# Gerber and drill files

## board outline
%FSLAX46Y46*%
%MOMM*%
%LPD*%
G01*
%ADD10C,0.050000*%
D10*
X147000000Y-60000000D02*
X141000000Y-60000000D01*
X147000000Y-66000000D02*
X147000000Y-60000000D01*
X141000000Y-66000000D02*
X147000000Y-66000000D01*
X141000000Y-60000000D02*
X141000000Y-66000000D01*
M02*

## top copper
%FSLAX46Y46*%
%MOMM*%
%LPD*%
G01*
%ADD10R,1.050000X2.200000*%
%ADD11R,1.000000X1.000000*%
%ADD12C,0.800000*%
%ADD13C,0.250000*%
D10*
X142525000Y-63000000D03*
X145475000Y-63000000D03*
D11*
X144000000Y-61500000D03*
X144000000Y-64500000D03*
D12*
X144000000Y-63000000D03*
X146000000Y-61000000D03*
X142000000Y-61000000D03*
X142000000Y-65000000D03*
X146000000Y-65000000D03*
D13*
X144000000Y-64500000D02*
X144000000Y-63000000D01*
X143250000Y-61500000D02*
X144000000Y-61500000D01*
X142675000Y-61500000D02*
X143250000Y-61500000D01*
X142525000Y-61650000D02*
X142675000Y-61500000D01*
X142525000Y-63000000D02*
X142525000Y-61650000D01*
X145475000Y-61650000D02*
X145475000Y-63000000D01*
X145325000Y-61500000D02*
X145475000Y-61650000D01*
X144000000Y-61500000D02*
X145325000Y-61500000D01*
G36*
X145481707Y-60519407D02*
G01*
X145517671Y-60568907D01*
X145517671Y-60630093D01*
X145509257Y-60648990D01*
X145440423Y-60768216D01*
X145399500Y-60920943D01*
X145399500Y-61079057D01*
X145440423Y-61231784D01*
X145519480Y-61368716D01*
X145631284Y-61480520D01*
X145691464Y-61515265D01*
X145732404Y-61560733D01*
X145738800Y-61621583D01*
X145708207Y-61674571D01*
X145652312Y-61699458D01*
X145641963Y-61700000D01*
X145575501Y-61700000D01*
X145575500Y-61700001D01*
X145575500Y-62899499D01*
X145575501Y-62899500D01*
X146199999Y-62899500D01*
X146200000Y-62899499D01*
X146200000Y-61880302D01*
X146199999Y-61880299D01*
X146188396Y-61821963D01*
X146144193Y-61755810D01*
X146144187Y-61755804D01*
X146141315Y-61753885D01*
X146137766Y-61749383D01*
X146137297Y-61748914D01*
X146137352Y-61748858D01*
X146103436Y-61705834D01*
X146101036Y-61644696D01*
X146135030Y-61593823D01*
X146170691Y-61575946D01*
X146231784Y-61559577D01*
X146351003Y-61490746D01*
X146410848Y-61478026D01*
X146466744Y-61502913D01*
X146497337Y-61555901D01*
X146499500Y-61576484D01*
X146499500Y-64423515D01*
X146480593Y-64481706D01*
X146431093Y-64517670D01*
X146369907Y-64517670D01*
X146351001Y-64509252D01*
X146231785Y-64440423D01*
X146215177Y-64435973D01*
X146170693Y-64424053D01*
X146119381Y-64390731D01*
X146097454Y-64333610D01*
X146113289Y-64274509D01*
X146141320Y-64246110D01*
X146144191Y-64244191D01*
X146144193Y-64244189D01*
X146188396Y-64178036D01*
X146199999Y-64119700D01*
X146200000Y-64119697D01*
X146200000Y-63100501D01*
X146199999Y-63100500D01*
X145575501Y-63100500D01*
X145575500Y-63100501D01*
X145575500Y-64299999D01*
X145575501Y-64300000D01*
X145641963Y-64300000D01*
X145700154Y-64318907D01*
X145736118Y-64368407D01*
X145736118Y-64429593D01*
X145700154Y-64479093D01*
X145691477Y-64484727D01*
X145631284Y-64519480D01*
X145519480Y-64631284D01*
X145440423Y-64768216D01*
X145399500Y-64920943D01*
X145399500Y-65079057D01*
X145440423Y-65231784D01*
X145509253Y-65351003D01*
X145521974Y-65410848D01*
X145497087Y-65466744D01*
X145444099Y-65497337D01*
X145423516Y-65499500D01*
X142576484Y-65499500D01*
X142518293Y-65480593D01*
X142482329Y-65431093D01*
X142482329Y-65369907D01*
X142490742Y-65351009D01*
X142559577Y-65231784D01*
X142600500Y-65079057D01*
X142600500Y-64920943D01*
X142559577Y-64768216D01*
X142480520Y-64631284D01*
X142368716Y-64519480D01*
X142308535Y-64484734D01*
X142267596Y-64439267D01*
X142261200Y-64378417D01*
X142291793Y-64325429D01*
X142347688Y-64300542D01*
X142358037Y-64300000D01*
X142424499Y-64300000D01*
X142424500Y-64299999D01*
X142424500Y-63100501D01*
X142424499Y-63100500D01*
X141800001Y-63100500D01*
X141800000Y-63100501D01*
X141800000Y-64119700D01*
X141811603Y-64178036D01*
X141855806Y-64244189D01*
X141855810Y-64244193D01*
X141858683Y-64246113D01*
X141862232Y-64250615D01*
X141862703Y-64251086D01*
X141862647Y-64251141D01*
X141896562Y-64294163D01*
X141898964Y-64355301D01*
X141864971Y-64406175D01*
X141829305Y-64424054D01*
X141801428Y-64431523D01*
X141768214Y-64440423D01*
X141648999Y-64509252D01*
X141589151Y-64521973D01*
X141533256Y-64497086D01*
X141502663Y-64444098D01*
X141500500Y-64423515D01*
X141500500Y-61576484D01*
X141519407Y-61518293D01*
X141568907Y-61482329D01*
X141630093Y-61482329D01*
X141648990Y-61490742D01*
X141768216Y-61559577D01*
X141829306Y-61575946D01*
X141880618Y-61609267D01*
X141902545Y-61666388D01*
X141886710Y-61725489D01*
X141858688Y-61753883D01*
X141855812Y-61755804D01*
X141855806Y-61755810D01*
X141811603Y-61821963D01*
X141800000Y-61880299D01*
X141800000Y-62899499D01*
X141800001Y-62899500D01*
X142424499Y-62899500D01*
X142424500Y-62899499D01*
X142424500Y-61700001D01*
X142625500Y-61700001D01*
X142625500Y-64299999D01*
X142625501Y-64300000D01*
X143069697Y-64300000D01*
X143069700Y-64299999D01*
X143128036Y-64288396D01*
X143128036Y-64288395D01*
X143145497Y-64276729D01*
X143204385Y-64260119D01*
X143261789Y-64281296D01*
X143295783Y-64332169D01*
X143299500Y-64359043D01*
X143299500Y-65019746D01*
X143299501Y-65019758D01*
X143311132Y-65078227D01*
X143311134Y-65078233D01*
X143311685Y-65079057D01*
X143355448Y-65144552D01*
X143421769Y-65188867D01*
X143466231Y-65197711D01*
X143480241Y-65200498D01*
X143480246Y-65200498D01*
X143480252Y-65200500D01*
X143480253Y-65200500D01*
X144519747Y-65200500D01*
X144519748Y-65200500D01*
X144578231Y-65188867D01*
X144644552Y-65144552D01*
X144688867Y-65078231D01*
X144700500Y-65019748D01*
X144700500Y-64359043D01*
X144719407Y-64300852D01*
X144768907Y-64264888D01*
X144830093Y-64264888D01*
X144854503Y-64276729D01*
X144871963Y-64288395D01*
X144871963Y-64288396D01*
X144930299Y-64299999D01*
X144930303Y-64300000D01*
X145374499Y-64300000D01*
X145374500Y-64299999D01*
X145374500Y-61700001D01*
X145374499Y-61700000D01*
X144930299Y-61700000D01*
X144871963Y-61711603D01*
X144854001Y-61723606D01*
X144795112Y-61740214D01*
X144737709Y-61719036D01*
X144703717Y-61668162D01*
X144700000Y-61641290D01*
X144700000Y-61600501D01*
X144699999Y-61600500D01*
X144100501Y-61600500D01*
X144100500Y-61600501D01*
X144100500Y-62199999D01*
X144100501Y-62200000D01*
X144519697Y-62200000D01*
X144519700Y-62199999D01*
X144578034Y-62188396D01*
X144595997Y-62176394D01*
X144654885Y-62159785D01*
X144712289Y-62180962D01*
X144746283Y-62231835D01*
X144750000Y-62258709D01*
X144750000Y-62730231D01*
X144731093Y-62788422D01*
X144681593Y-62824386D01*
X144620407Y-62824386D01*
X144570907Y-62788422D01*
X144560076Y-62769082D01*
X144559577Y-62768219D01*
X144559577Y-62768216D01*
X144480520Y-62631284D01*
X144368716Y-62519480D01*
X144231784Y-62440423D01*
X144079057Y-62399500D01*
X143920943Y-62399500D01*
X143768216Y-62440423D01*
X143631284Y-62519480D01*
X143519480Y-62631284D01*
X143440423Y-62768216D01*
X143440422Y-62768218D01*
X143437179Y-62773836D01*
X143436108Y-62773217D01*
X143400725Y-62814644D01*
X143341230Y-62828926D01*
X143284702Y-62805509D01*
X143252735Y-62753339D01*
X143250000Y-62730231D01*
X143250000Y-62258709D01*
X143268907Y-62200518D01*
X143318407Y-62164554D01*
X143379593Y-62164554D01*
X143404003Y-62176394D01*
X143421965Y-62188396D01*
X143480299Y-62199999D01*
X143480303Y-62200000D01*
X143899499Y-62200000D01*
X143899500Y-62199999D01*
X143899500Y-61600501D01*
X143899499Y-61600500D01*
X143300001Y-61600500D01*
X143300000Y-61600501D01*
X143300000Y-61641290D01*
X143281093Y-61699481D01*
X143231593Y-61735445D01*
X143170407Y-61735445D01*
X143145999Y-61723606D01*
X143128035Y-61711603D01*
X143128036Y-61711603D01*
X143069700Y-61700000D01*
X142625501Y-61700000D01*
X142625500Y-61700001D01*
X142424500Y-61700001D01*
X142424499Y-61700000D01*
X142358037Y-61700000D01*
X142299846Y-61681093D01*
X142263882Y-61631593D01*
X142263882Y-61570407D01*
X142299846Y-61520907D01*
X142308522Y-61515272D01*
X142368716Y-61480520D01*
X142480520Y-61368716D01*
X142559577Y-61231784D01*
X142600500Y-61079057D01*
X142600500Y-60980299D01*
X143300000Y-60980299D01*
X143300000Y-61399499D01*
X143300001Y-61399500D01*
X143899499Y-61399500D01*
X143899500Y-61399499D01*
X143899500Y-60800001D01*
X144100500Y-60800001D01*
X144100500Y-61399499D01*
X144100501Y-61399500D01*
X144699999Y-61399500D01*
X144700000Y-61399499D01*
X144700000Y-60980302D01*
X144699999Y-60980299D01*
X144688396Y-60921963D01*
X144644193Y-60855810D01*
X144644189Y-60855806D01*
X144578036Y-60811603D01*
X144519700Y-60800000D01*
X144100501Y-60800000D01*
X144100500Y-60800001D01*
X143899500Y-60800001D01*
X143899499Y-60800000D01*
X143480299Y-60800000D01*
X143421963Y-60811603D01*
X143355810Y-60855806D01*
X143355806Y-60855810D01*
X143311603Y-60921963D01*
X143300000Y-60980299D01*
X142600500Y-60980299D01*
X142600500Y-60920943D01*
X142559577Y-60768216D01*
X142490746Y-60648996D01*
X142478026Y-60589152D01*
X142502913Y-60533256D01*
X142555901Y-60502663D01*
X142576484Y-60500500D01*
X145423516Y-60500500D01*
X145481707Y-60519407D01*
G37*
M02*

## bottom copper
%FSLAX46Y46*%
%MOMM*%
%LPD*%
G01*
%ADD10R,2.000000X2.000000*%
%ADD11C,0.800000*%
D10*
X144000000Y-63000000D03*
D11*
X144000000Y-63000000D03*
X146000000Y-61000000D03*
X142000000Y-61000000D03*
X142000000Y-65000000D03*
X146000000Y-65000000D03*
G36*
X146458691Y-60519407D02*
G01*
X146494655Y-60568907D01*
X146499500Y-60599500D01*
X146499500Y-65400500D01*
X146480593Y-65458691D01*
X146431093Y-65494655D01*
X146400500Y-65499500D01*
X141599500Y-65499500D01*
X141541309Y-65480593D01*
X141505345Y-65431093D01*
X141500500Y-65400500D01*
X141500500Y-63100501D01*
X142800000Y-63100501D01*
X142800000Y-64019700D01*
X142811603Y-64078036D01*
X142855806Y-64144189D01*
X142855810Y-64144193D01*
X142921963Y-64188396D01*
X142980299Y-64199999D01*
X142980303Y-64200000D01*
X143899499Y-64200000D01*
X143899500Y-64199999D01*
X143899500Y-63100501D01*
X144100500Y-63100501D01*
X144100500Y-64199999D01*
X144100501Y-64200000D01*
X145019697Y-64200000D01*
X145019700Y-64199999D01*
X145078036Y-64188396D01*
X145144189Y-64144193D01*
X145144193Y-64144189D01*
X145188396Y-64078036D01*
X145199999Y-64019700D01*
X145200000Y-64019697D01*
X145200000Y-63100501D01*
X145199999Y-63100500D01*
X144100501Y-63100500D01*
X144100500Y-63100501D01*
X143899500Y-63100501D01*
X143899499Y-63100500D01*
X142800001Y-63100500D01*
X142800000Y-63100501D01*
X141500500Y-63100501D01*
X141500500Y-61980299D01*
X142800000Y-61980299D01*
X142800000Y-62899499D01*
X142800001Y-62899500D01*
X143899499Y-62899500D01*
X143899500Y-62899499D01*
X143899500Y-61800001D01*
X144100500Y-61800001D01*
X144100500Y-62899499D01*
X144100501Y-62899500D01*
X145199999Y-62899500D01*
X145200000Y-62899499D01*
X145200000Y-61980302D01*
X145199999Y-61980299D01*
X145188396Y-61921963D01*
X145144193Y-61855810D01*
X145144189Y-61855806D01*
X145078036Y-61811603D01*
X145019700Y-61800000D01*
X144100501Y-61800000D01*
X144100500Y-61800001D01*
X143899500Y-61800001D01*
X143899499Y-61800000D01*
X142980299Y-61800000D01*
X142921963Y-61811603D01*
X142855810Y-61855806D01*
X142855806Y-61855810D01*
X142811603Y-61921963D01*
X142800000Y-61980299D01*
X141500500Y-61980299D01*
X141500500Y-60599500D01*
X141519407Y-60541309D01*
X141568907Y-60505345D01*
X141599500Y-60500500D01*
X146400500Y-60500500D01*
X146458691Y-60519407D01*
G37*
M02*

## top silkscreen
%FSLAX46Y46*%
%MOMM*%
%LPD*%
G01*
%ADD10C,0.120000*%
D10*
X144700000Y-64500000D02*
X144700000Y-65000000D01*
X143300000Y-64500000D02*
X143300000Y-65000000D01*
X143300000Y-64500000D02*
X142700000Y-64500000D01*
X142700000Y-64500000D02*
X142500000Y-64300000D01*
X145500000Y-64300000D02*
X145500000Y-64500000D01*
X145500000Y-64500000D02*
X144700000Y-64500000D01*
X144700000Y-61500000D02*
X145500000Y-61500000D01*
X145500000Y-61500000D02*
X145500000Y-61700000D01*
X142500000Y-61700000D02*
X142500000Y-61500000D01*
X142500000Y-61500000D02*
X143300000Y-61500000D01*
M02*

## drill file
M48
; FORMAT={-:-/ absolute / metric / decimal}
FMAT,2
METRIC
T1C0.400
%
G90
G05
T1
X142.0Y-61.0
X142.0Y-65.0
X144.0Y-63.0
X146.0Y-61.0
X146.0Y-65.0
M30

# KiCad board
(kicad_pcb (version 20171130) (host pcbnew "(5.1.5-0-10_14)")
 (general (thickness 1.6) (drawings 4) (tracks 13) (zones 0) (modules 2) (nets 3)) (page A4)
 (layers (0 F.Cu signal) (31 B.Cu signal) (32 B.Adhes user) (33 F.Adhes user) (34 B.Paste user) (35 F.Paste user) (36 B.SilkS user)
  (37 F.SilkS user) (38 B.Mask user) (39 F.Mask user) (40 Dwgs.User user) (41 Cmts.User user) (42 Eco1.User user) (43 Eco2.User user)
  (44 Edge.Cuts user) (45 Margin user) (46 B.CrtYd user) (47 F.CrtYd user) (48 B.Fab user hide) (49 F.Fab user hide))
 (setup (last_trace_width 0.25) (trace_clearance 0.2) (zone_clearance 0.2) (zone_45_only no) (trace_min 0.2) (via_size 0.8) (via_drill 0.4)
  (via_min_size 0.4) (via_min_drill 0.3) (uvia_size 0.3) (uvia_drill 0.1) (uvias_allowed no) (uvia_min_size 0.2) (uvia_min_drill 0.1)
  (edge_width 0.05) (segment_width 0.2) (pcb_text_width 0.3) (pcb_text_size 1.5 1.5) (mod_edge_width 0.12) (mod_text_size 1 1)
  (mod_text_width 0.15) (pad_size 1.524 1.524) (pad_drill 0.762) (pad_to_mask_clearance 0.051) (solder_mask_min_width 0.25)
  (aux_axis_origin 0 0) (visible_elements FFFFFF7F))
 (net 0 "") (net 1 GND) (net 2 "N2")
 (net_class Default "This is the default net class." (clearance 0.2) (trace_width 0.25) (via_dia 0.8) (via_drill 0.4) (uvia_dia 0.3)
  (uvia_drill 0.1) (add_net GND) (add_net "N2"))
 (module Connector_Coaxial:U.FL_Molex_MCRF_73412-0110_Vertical (layer F.Cu) (at 144 63)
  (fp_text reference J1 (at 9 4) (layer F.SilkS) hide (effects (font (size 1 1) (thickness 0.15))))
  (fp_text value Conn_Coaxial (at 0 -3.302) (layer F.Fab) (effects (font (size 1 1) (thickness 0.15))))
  (fp_line (start 0.7 1.5) (end 0.7 2) (layer F.SilkS) (width 0.12))
  (fp_line (start -0.7 1.5) (end -0.7 2) (layer F.SilkS) (width 0.12))
  (fp_line (start -0.7 1.5) (end -1.3 1.5) (layer F.SilkS) (width 0.12))
  (fp_line (start -1.3 1.5) (end -1.5 1.3) (layer F.SilkS) (width 0.12))
  (fp_line (start 1.5 1.3) (end 1.5 1.5) (layer F.SilkS) (width 0.12))
  (fp_line (start 1.5 1.5) (end 0.7 1.5) (layer F.SilkS) (width 0.12))
  (fp_line (start 0.7 -1.5) (end 1.5 -1.5) (layer F.SilkS) (width 0.12))
  (fp_line (start 1.5 -1.5) (end 1.5 -1.3) (layer F.SilkS) (width 0.12))
  (fp_line (start -1.5 -1.3) (end -1.5 -1.5) (layer F.SilkS) (width 0.12))
  (fp_line (start -1.5 -1.5) (end -0.7 -1.5) (layer F.SilkS) (width 0.12))
  (pad 2 smd rect (at -1.475 0) (size 1.05 2.2) (layers F.Cu F.Paste F.Mask) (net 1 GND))
  (pad 2 smd rect (at 1.475 0) (size 1.05 2.2) (layers F.Cu F.Paste F.Mask) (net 1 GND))
  (pad 2 smd rect (at 0 -1.5) (size 1 1) (layers F.Cu F.Paste F.Mask) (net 1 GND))
  (pad 1 smd rect (at 0 1.5) (size 1 1) (layers F.Cu F.Paste F.Mask) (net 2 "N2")))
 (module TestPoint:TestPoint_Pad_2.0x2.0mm (layer B.Cu) (at 144 63)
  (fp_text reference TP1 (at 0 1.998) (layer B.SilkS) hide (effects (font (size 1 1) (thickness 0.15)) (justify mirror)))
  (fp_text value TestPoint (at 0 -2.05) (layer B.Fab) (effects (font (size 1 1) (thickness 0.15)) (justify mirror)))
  (pad 1 smd rect (at 0 0) (size 2 2) (layers B.Cu B.Mask) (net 2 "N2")))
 (gr_line (start 147 60) (end 141 60) (layer Edge.Cuts) (width 0.05))
 (gr_line (start 147 66) (end 147 60) (layer Edge.Cuts) (width 0.05))
 (gr_line (start 141 66) (end 147 66) (layer Edge.Cuts) (width 0.05))
 (gr_line (start 141 60) (end 141 66) (layer Edge.Cuts) (width 0.05))
 (via (at 144 63) (size 0.8) (drill 0.4) (layers F.Cu B.Cu) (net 2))
 (segment (start 144 64.5) (end 144 63) (width 0.25) (layer F.Cu) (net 2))
 (via (at 146 61) (size 0.8) (drill 0.4) (layers F.Cu B.Cu) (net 2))
 (via (at 142 61) (size 0.8) (drill 0.4) (layers F.Cu B.Cu) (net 2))
 (via (at 142 65) (size 0.8) (drill 0.4) (layers F.Cu B.Cu) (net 2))
 (via (at 146 65) (size 0.8) (drill 0.4) (layers F.Cu B.Cu) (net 2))
 (segment (start 143.25 61.5) (end 144 61.5) (width 0.25) (layer F.Cu) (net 1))
 (segment (start 142.675 61.5) (end 143.25 61.5) (width 0.25) (layer F.Cu) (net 1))
 (segment (start 142.525 61.65) (end 142.675 61.5) (width 0.25) (layer F.Cu) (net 1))
 (segment (start 142.525 63) (end 142.525 61.65) (width 0.25) (layer F.Cu) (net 1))
 (segment (start 145.475 61.65) (end 145.475 63) (width 0.25) (layer F.Cu) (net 1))
 (segment (start 145.325 61.5) (end 145.475 61.65) (width 0.25) (layer F.Cu) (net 1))
 (segment (start 144 61.5) (end 145.325 61.5) (width 0.25) (layer F.Cu) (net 1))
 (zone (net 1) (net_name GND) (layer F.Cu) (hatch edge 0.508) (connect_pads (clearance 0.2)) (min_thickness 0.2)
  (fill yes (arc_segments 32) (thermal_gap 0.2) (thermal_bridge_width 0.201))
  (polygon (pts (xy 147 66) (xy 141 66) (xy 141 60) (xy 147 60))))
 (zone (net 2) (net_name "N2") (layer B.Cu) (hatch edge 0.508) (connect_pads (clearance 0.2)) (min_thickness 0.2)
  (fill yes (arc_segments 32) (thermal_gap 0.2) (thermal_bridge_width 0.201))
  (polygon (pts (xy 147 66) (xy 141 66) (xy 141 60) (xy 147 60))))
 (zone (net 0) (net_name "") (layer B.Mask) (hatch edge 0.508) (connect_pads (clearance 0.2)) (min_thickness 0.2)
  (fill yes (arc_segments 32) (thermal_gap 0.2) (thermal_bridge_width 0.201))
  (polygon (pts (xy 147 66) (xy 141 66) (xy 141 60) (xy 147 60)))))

